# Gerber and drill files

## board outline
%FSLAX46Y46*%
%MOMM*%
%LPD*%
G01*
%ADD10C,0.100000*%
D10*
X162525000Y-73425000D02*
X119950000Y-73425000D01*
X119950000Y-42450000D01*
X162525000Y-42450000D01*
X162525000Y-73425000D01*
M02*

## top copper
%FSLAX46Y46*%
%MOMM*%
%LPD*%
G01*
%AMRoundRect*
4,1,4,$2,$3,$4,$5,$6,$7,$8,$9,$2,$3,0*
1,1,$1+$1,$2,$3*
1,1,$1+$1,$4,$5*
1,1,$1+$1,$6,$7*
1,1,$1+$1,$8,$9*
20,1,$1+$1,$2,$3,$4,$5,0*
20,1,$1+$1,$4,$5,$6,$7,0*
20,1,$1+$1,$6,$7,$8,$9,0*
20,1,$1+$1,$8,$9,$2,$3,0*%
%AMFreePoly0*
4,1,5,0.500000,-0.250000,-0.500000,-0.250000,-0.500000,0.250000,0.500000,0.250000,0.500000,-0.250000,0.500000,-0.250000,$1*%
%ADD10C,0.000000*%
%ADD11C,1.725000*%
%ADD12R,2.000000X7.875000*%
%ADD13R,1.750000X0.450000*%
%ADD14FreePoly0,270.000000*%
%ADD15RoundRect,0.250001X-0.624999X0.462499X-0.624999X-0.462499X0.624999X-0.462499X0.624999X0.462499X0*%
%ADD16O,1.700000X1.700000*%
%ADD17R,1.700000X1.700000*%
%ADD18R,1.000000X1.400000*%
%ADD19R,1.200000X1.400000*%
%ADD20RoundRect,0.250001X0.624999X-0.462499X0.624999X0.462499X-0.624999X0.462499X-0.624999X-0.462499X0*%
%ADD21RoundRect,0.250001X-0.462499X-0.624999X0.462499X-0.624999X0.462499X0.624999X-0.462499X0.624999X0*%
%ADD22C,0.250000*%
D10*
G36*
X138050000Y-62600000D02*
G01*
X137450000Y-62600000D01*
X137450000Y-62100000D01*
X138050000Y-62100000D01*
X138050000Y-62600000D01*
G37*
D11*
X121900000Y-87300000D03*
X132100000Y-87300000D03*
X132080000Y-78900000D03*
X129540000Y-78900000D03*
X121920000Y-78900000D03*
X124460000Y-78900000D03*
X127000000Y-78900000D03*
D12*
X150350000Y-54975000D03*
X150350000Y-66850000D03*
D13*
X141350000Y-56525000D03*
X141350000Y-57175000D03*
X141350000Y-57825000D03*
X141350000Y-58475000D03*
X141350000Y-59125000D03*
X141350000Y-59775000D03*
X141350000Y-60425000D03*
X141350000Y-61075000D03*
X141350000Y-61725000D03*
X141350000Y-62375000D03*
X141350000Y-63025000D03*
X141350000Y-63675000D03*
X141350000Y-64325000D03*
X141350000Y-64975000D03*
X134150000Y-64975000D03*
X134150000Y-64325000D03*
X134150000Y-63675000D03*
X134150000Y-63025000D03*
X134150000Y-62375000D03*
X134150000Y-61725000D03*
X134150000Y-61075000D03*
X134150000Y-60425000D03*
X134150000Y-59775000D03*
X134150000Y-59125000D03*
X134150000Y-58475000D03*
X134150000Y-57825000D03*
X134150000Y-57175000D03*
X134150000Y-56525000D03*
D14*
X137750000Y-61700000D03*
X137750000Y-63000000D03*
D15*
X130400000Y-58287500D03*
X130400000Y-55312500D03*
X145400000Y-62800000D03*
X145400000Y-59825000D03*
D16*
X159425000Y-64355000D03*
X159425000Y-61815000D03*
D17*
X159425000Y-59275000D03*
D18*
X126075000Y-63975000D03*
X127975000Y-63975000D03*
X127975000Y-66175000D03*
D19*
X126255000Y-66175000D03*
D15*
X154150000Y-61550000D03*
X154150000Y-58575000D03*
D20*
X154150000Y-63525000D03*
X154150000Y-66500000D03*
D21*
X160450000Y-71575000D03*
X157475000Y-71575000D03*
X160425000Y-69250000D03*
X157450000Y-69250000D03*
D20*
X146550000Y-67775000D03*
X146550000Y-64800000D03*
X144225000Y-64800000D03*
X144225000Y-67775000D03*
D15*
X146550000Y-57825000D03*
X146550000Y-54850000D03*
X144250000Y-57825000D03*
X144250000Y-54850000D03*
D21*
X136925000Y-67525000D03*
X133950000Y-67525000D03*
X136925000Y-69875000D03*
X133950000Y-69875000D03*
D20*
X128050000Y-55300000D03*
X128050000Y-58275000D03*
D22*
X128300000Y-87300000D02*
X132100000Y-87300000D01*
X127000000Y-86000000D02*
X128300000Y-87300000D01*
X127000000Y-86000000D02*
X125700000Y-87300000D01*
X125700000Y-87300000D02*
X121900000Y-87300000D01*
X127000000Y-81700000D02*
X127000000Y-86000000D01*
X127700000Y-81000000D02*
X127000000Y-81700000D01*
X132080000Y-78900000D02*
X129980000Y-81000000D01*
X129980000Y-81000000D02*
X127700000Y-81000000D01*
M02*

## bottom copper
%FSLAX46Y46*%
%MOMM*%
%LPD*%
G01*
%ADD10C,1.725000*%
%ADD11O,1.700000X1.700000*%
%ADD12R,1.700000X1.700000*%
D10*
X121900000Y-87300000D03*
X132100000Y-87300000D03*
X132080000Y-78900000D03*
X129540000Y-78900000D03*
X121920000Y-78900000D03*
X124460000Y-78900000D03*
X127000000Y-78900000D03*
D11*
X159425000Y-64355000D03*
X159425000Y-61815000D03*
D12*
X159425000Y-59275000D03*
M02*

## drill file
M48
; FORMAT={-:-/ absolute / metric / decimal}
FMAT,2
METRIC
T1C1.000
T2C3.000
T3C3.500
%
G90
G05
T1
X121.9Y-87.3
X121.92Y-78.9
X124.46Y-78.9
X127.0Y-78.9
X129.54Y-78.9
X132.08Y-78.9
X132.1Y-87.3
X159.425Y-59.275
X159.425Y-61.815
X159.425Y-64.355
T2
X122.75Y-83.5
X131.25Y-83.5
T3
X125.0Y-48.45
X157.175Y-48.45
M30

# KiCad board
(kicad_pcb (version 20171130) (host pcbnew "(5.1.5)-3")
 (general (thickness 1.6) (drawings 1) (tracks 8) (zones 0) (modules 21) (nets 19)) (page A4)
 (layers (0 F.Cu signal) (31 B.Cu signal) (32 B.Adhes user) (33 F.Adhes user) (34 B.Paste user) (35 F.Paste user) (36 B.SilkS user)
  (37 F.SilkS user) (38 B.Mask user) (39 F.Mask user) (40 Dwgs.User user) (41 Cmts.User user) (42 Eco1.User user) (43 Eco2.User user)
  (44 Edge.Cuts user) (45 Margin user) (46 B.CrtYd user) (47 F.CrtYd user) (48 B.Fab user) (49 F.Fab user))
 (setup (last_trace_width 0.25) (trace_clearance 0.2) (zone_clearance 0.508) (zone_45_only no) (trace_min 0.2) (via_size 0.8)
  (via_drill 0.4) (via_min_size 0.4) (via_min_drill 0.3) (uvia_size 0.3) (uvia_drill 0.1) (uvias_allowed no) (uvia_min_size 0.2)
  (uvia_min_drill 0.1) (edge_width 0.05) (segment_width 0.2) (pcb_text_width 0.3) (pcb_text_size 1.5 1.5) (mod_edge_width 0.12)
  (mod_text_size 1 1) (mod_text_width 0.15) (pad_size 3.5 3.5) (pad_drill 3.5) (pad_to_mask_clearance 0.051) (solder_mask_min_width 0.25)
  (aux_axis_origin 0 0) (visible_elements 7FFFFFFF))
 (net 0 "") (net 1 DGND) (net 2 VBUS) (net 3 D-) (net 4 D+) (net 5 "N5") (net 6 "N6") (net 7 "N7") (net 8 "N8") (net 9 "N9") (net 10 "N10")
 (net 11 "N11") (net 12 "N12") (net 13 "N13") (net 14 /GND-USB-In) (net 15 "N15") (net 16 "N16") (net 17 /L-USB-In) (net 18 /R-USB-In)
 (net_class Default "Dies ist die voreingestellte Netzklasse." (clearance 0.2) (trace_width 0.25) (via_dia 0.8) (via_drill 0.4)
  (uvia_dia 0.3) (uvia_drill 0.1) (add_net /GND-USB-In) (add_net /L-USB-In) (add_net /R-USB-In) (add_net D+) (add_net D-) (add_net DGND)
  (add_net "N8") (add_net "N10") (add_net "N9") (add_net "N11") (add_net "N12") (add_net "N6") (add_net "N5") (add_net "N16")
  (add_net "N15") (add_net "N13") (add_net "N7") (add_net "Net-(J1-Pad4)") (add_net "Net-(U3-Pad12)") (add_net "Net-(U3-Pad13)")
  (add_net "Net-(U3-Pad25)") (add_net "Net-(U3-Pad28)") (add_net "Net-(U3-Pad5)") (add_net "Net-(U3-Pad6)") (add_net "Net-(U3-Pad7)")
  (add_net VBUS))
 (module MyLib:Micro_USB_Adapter (layer F.Cu) (at 127 84.65 180)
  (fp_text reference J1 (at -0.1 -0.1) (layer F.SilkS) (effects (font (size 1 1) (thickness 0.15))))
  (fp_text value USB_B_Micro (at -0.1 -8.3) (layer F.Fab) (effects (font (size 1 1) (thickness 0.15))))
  (pad 6 thru_hole circle (at 5.1 -2.65 180) (size 1.725 1.725) (drill 1) (layers *.Cu *.Mask) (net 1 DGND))
  (pad 6 thru_hole circle (at -5.1 -2.65 180) (size 1.725 1.725) (drill 1) (layers *.Cu *.Mask) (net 1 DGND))
  (pad "" np_thru_hole circle (at 4.25 1.15 180) (size 3 3) (drill 3) (layers *.Cu *.Mask))
  (pad "" np_thru_hole circle (at -4.25 1.15 180) (size 3 3) (drill 3) (layers *.Cu *.Mask))
  (pad 5 thru_hole circle (at -5.08 5.75 180) (size 1.725 1.725) (drill 1) (layers *.Cu *.Mask) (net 1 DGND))
  (pad 4 thru_hole circle (at -2.54 5.75 180) (size 1.725 1.725) (drill 1) (layers *.Cu *.Mask))
  (pad 1 thru_hole circle (at 5.08 5.75 180) (size 1.725 1.725) (drill 1) (layers *.Cu *.Mask) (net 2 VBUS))
  (pad 2 thru_hole circle (at 2.54 5.75 180) (size 1.725 1.725) (drill 1) (layers *.Cu *.Mask) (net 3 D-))
  (pad 3 thru_hole circle (at 0 5.75 180) (size 1.725 1.725) (drill 1) (layers *.Cu *.Mask) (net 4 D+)))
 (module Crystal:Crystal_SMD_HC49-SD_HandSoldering (layer F.Cu) (at 150.35 60.9125 90)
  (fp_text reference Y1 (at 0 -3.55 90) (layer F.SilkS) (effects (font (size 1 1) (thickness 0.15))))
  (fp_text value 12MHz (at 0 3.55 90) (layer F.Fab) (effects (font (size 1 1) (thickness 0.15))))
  (pad 2 smd rect (at 5.9375 0 90) (size 7.875 2) (layers F.Cu F.Paste F.Mask) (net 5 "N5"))
  (pad 1 smd rect (at -5.9375 0 90) (size 7.875 2) (layers F.Cu F.Paste F.Mask) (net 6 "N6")))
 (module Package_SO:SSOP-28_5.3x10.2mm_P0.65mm (layer F.Cu) (at 137.75 60.75)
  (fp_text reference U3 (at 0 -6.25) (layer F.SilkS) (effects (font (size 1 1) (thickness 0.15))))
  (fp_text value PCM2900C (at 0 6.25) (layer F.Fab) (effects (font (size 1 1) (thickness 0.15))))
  (pad 28 smd rect (at 3.6 -4.225) (size 1.75 0.45) (layers F.Cu F.Paste F.Mask))
  (pad 27 smd rect (at 3.6 -3.575) (size 1.75 0.45) (layers F.Cu F.Paste F.Mask) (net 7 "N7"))
  (pad 26 smd rect (at 3.6 -2.925) (size 1.75 0.45) (layers F.Cu F.Paste F.Mask) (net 1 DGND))
  (pad 25 smd rect (at 3.6 -2.275) (size 1.75 0.45) (layers F.Cu F.Paste F.Mask))
  (pad 24 smd rect (at 3.6 -1.625) (size 1.75 0.45) (layers F.Cu F.Paste F.Mask) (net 1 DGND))
  (pad 23 smd rect (at 3.6 -0.975) (size 1.75 0.45) (layers F.Cu F.Paste F.Mask) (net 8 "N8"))
  (pad 22 smd rect (at 3.6 -0.325) (size 1.75 0.45) (layers F.Cu F.Paste F.Mask) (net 1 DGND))
  (pad 21 smd rect (at 3.6 0.325) (size 1.75 0.45) (layers F.Cu F.Paste F.Mask) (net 5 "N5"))
  (pad 20 smd rect (at 3.6 0.975) (size 1.75 0.45) (layers F.Cu F.Paste F.Mask) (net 6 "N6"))
  (pad 19 smd rect (at 3.6 1.625) (size 1.75 0.45) (layers F.Cu F.Paste F.Mask) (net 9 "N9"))
  (pad 18 smd rect (at 3.6 2.275) (size 1.75 0.45) (layers F.Cu F.Paste F.Mask) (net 1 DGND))
  (pad 17 smd rect (at 3.6 2.925) (size 1.75 0.45) (layers F.Cu F.Paste F.Mask) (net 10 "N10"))
  (pad 16 smd rect (at 3.6 3.575) (size 1.75 0.45) (layers F.Cu F.Paste F.Mask) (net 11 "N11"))
  (pad 15 smd rect (at 3.6 4.225) (size 1.75 0.45) (layers F.Cu F.Paste F.Mask) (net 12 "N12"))
  (pad 14 smd rect (at -3.6 4.225) (size 1.75 0.45) (layers F.Cu F.Paste F.Mask) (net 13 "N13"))
  (pad 13 smd rect (at -3.6 3.575) (size 1.75 0.45) (layers F.Cu F.Paste F.Mask))
  (pad 12 smd rect (at -3.6 2.925) (size 1.75 0.45) (layers F.Cu F.Paste F.Mask))
  (pad 11 smd rect (at -3.6 2.275) (size 1.75 0.45) (layers F.Cu F.Paste F.Mask) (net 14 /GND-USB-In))
  (pad 10 smd rect (at -3.6 1.625) (size 1.75 0.45) (layers F.Cu F.Paste F.Mask) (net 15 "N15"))
  (pad 9 smd rect (at -3.6 0.975) (size 1.75 0.45) (layers F.Cu F.Paste F.Mask) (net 7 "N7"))
  (pad 8 smd rect (at -3.6 0.325) (size 1.75 0.45) (layers F.Cu F.Paste F.Mask) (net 7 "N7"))
  (pad 7 smd rect (at -3.6 -0.325) (size 1.75 0.45) (layers F.Cu F.Paste F.Mask))
  (pad 6 smd rect (at -3.6 -0.975) (size 1.75 0.45) (layers F.Cu F.Paste F.Mask))
  (pad 5 smd rect (at -3.6 -1.625) (size 1.75 0.45) (layers F.Cu F.Paste F.Mask))
  (pad 4 smd rect (at -3.6 -2.275) (size 1.75 0.45) (layers F.Cu F.Paste F.Mask) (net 1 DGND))
  (pad 3 smd rect (at -3.6 -2.925) (size 1.75 0.45) (layers F.Cu F.Paste F.Mask) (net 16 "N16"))
  (pad 2 smd rect (at -3.6 -3.575) (size 1.75 0.45) (layers F.Cu F.Paste F.Mask) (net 3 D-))
  (pad 1 smd rect (at -3.6 -4.225) (size 1.75 0.45) (layers F.Cu F.Paste F.Mask) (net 4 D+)))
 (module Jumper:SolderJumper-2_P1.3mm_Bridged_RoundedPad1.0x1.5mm (layer F.Cu) (at 137.75 62.35 270)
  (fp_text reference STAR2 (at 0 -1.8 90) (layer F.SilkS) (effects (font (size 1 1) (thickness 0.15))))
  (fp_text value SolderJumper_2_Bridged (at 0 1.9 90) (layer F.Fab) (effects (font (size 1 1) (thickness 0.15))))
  (fp_poly (pts (xy 0.25 -0.3) (xy -0.25 -0.3) (xy -0.25 0.3) (xy 0.25 0.3)) (layer F.Cu) (width 0))
  (pad 1 smd custom (at -0.65 0 270) (size 1 0.5) (layers F.Cu F.Mask) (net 1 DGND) (zone_connect 2)
   (options (clearance outline) (anchor rect)) (primitives))
  (pad 2 smd custom (at 0.65 0 270) (size 1 0.5) (layers F.Cu F.Mask) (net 14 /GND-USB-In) (zone_connect 2)
   (options (clearance outline) (anchor rect)) (primitives)))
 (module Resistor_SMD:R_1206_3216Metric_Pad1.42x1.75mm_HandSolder (layer F.Cu) (at 130.4 56.8 270)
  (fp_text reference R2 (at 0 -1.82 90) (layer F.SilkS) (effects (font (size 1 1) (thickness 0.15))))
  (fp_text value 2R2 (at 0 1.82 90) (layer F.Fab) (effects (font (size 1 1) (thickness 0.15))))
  (pad 2 smd roundrect (at 1.4875 0 270) (size 1.425 1.75) (layers F.Cu F.Paste F.Mask) (roundrect_rratio 0.175439) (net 16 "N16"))
  (pad 1 smd roundrect (at -1.4875 0 270) (size 1.425 1.75) (layers F.Cu F.Paste F.Mask) (roundrect_rratio 0.175439) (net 2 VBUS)))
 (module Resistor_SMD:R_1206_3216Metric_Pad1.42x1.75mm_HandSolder (layer F.Cu) (at 145.4 61.3125 270)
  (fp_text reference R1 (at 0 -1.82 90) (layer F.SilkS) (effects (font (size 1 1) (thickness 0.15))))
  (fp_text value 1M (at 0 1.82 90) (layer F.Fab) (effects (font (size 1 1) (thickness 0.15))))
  (pad 2 smd roundrect (at 1.4875 0 270) (size 1.425 1.75) (layers F.Cu F.Paste F.Mask) (roundrect_rratio 0.175439) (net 6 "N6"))
  (pad 1 smd roundrect (at -1.4875 0 270) (size 1.425 1.75) (layers F.Cu F.Paste F.Mask) (roundrect_rratio 0.175439) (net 5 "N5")))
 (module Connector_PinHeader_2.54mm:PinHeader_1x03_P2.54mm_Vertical (layer F.Cu) (at 159.425 59.275)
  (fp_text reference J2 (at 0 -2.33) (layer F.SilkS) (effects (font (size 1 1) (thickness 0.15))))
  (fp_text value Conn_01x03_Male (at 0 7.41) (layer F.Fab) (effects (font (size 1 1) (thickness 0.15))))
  (pad 3 thru_hole oval (at 0 5.08) (size 1.7 1.7) (drill 1) (layers *.Cu *.Mask) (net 14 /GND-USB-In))
  (pad 2 thru_hole oval (at 0 2.54) (size 1.7 1.7) (drill 1) (layers *.Cu *.Mask) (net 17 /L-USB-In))
  (pad 1 thru_hole rect (at 0 0) (size 1.7 1.7) (drill 1) (layers *.Cu *.Mask) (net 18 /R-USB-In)))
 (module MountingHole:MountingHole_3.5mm (layer F.Cu) (at 157.175 48.45)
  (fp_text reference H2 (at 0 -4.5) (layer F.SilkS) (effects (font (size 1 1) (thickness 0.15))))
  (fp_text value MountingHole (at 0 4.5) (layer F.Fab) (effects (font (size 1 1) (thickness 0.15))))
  (pad 1 np_thru_hole circle (at 0 0) (size 3.5 3.5) (drill 3.5) (layers *.Cu *.Mask)))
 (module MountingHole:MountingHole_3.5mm (layer F.Cu) (at 125 48.45)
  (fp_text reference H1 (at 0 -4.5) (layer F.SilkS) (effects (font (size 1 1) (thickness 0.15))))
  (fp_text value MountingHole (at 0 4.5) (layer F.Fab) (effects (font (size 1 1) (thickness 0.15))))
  (pad 1 np_thru_hole circle (at 0 0) (size 3.5 3.5) (drill 3.5) (layers *.Cu *.Mask)))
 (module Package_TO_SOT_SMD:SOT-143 (layer F.Cu) (at 127.025 65.075 90)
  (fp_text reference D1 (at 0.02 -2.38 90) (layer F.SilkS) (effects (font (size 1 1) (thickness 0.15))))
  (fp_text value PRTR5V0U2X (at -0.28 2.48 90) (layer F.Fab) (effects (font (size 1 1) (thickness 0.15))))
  (pad 4 smd rect (at 1.1 -0.95) (size 1 1.4) (layers F.Cu F.Paste F.Mask) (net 2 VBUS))
  (pad 3 smd rect (at 1.1 0.95) (size 1 1.4) (layers F.Cu F.Paste F.Mask) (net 4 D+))
  (pad 2 smd rect (at -1.1 0.95) (size 1 1.4) (layers F.Cu F.Paste F.Mask) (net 3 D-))
  (pad 1 smd rect (at -1.1 -0.77) (size 1.2 1.4) (layers F.Cu F.Paste F.Mask) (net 1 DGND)))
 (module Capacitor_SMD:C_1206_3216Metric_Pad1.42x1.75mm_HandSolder (layer F.Cu) (at 154.15 60.0625 270)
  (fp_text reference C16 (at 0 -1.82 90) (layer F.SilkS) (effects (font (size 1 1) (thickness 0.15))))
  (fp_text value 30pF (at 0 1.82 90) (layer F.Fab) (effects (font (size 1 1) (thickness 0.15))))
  (pad 2 smd roundrect (at 1.4875 0 270) (size 1.425 1.75) (layers F.Cu F.Paste F.Mask) (roundrect_rratio 0.175439) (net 1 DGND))
  (pad 1 smd roundrect (at -1.4875 0 270) (size 1.425 1.75) (layers F.Cu F.Paste F.Mask) (roundrect_rratio 0.175439) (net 5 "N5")))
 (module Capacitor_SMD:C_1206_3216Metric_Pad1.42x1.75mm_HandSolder (layer F.Cu) (at 154.15 65.0125 90)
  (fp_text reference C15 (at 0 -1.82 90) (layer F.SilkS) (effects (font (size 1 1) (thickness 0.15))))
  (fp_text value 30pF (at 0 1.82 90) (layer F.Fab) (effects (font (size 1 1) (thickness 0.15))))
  (pad 2 smd roundrect (at 1.4875 0 90) (size 1.425 1.75) (layers F.Cu F.Paste F.Mask) (roundrect_rratio 0.175439) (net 1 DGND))
  (pad 1 smd roundrect (at -1.4875 0 90) (size 1.425 1.75) (layers F.Cu F.Paste F.Mask) (roundrect_rratio 0.175439) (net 6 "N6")))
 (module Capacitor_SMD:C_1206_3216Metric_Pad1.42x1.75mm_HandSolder (layer F.Cu) (at 158.9625 71.575)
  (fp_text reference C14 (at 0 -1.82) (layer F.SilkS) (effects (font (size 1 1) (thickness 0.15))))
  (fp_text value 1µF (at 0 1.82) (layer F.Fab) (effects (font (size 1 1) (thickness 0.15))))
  (pad 2 smd roundrect (at 1.4875 0) (size 1.425 1.75) (layers F.Cu F.Paste F.Mask) (roundrect_rratio 0.175439) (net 17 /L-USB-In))
  (pad 1 smd roundrect (at -1.4875 0) (size 1.425 1.75) (layers F.Cu F.Paste F.Mask) (roundrect_rratio 0.175439) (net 12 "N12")))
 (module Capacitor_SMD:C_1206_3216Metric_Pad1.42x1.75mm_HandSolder (layer F.Cu) (at 158.9375 69.25)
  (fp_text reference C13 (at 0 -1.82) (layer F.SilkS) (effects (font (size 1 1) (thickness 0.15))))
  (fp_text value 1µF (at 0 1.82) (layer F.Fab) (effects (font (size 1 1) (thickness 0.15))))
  (pad 2 smd roundrect (at 1.4875 0) (size 1.425 1.75) (layers F.Cu F.Paste F.Mask) (roundrect_rratio 0.175439) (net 18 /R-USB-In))
  (pad 1 smd roundrect (at -1.4875 0) (size 1.425 1.75) (layers F.Cu F.Paste F.Mask) (roundrect_rratio 0.175439) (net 11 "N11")))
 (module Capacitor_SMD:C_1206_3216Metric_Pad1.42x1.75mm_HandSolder (layer F.Cu) (at 146.55 66.2875 90)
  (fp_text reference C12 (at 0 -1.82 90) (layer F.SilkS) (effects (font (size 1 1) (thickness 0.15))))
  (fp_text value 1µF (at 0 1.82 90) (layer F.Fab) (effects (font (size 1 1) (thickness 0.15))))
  (pad 1 smd roundrect (at -1.4875 0 90) (size 1.425 1.75) (layers F.Cu F.Paste F.Mask) (roundrect_rratio 0.175439) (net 9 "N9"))
  (pad 2 smd roundrect (at 1.4875 0 90) (size 1.425 1.75) (layers F.Cu F.Paste F.Mask) (roundrect_rratio 0.175439) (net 1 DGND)))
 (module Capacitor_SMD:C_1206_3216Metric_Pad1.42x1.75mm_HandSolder (layer F.Cu) (at 144.225 66.2875 90)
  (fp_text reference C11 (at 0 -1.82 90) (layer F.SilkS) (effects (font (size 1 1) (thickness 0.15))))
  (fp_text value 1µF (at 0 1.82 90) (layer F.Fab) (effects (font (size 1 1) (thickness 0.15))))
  (pad 2 smd roundrect (at 1.4875 0 90) (size 1.425 1.75) (layers F.Cu F.Paste F.Mask) (roundrect_rratio 0.175439) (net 1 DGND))
  (pad 1 smd roundrect (at -1.4875 0 90) (size 1.425 1.75) (layers F.Cu F.Paste F.Mask) (roundrect_rratio 0.175439) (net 10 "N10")))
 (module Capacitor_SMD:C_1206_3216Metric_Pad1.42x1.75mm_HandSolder (layer F.Cu) (at 146.55 56.3375 270)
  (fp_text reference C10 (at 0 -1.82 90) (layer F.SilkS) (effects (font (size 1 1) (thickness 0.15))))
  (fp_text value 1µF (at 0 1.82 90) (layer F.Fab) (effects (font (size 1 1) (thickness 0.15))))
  (pad 2 smd roundrect (at 1.4875 0 270) (size 1.425 1.75) (layers F.Cu F.Paste F.Mask) (roundrect_rratio 0.175439) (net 1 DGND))
  (pad 1 smd roundrect (at -1.4875 0 270) (size 1.425 1.75) (layers F.Cu F.Paste F.Mask) (roundrect_rratio 0.175439) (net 8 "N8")))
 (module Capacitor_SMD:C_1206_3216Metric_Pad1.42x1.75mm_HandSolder (layer F.Cu) (at 144.25 56.3375 270)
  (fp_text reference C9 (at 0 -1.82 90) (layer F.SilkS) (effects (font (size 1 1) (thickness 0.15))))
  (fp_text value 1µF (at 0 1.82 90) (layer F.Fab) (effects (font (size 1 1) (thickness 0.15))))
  (pad 2 smd roundrect (at 1.4875 0 270) (size 1.425 1.75) (layers F.Cu F.Paste F.Mask) (roundrect_rratio 0.175439) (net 1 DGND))
  (pad 1 smd roundrect (at -1.4875 0 270) (size 1.425 1.75) (layers F.Cu F.Paste F.Mask) (roundrect_rratio 0.175439) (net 7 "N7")))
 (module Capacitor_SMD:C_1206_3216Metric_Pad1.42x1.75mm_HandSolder (layer F.Cu) (at 135.4375 67.525)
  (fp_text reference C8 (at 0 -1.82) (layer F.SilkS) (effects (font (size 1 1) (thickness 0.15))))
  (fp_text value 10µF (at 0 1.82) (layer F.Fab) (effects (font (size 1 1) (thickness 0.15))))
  (pad 2 smd roundrect (at 1.4875 0) (size 1.425 1.75) (layers F.Cu F.Paste F.Mask) (roundrect_rratio 0.175439) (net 1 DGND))
  (pad 1 smd roundrect (at -1.4875 0) (size 1.425 1.75) (layers F.Cu F.Paste F.Mask) (roundrect_rratio 0.175439) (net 13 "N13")))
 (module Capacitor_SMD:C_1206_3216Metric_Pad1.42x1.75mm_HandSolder (layer F.Cu) (at 135.4375 69.875)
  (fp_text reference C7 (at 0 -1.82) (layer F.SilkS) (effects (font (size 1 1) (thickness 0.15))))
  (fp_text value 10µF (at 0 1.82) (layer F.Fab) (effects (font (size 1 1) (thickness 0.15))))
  (pad 2 smd roundrect (at 1.4875 0) (size 1.425 1.75) (layers F.Cu F.Paste F.Mask) (roundrect_rratio 0.175439) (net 1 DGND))
  (pad 1 smd roundrect (at -1.4875 0) (size 1.425 1.75) (layers F.Cu F.Paste F.Mask) (roundrect_rratio 0.175439) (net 15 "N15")))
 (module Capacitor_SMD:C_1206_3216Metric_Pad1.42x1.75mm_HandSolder (layer F.Cu) (at 128.05 56.7875 90)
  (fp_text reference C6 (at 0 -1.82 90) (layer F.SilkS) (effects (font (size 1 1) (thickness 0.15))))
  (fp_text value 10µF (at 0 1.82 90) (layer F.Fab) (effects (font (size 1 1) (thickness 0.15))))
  (pad 2 smd roundrect (at 1.4875 0 90) (size 1.425 1.75) (layers F.Cu F.Paste F.Mask) (roundrect_rratio 0.175439) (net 1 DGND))
  (pad 1 smd roundrect (at -1.4875 0 90) (size 1.425 1.75) (layers F.Cu F.Paste F.Mask) (roundrect_rratio 0.175439) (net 16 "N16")))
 (gr_poly (pts (xy 162.525 73.425) (xy 119.95 73.425) (xy 119.95 42.45) (xy 162.525 42.45)) (layer Edge.Cuts) (width 0.1))
 (segment (start 128.3 87.3) (end 132.1 87.3) (width 0.25) (layer F.Cu) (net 1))
 (segment (start 127 86) (end 128.3 87.3) (width 0.25) (layer F.Cu) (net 1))
 (segment (start 127 86) (end 125.7 87.3) (width 0.25) (layer F.Cu) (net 1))
 (segment (start 125.7 87.3) (end 121.9 87.3) (width 0.25) (layer F.Cu) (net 1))
 (segment (start 127 81.7) (end 127 86) (width 0.25) (layer F.Cu) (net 1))
 (segment (start 127.7 81) (end 127 81.7) (width 0.25) (layer F.Cu) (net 1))
 (segment (start 132.08 78.9) (end 129.98 81) (width 0.25) (layer F.Cu) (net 1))
 (segment (start 129.98 81) (end 127.7 81) (width 0.25) (layer F.Cu) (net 1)))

